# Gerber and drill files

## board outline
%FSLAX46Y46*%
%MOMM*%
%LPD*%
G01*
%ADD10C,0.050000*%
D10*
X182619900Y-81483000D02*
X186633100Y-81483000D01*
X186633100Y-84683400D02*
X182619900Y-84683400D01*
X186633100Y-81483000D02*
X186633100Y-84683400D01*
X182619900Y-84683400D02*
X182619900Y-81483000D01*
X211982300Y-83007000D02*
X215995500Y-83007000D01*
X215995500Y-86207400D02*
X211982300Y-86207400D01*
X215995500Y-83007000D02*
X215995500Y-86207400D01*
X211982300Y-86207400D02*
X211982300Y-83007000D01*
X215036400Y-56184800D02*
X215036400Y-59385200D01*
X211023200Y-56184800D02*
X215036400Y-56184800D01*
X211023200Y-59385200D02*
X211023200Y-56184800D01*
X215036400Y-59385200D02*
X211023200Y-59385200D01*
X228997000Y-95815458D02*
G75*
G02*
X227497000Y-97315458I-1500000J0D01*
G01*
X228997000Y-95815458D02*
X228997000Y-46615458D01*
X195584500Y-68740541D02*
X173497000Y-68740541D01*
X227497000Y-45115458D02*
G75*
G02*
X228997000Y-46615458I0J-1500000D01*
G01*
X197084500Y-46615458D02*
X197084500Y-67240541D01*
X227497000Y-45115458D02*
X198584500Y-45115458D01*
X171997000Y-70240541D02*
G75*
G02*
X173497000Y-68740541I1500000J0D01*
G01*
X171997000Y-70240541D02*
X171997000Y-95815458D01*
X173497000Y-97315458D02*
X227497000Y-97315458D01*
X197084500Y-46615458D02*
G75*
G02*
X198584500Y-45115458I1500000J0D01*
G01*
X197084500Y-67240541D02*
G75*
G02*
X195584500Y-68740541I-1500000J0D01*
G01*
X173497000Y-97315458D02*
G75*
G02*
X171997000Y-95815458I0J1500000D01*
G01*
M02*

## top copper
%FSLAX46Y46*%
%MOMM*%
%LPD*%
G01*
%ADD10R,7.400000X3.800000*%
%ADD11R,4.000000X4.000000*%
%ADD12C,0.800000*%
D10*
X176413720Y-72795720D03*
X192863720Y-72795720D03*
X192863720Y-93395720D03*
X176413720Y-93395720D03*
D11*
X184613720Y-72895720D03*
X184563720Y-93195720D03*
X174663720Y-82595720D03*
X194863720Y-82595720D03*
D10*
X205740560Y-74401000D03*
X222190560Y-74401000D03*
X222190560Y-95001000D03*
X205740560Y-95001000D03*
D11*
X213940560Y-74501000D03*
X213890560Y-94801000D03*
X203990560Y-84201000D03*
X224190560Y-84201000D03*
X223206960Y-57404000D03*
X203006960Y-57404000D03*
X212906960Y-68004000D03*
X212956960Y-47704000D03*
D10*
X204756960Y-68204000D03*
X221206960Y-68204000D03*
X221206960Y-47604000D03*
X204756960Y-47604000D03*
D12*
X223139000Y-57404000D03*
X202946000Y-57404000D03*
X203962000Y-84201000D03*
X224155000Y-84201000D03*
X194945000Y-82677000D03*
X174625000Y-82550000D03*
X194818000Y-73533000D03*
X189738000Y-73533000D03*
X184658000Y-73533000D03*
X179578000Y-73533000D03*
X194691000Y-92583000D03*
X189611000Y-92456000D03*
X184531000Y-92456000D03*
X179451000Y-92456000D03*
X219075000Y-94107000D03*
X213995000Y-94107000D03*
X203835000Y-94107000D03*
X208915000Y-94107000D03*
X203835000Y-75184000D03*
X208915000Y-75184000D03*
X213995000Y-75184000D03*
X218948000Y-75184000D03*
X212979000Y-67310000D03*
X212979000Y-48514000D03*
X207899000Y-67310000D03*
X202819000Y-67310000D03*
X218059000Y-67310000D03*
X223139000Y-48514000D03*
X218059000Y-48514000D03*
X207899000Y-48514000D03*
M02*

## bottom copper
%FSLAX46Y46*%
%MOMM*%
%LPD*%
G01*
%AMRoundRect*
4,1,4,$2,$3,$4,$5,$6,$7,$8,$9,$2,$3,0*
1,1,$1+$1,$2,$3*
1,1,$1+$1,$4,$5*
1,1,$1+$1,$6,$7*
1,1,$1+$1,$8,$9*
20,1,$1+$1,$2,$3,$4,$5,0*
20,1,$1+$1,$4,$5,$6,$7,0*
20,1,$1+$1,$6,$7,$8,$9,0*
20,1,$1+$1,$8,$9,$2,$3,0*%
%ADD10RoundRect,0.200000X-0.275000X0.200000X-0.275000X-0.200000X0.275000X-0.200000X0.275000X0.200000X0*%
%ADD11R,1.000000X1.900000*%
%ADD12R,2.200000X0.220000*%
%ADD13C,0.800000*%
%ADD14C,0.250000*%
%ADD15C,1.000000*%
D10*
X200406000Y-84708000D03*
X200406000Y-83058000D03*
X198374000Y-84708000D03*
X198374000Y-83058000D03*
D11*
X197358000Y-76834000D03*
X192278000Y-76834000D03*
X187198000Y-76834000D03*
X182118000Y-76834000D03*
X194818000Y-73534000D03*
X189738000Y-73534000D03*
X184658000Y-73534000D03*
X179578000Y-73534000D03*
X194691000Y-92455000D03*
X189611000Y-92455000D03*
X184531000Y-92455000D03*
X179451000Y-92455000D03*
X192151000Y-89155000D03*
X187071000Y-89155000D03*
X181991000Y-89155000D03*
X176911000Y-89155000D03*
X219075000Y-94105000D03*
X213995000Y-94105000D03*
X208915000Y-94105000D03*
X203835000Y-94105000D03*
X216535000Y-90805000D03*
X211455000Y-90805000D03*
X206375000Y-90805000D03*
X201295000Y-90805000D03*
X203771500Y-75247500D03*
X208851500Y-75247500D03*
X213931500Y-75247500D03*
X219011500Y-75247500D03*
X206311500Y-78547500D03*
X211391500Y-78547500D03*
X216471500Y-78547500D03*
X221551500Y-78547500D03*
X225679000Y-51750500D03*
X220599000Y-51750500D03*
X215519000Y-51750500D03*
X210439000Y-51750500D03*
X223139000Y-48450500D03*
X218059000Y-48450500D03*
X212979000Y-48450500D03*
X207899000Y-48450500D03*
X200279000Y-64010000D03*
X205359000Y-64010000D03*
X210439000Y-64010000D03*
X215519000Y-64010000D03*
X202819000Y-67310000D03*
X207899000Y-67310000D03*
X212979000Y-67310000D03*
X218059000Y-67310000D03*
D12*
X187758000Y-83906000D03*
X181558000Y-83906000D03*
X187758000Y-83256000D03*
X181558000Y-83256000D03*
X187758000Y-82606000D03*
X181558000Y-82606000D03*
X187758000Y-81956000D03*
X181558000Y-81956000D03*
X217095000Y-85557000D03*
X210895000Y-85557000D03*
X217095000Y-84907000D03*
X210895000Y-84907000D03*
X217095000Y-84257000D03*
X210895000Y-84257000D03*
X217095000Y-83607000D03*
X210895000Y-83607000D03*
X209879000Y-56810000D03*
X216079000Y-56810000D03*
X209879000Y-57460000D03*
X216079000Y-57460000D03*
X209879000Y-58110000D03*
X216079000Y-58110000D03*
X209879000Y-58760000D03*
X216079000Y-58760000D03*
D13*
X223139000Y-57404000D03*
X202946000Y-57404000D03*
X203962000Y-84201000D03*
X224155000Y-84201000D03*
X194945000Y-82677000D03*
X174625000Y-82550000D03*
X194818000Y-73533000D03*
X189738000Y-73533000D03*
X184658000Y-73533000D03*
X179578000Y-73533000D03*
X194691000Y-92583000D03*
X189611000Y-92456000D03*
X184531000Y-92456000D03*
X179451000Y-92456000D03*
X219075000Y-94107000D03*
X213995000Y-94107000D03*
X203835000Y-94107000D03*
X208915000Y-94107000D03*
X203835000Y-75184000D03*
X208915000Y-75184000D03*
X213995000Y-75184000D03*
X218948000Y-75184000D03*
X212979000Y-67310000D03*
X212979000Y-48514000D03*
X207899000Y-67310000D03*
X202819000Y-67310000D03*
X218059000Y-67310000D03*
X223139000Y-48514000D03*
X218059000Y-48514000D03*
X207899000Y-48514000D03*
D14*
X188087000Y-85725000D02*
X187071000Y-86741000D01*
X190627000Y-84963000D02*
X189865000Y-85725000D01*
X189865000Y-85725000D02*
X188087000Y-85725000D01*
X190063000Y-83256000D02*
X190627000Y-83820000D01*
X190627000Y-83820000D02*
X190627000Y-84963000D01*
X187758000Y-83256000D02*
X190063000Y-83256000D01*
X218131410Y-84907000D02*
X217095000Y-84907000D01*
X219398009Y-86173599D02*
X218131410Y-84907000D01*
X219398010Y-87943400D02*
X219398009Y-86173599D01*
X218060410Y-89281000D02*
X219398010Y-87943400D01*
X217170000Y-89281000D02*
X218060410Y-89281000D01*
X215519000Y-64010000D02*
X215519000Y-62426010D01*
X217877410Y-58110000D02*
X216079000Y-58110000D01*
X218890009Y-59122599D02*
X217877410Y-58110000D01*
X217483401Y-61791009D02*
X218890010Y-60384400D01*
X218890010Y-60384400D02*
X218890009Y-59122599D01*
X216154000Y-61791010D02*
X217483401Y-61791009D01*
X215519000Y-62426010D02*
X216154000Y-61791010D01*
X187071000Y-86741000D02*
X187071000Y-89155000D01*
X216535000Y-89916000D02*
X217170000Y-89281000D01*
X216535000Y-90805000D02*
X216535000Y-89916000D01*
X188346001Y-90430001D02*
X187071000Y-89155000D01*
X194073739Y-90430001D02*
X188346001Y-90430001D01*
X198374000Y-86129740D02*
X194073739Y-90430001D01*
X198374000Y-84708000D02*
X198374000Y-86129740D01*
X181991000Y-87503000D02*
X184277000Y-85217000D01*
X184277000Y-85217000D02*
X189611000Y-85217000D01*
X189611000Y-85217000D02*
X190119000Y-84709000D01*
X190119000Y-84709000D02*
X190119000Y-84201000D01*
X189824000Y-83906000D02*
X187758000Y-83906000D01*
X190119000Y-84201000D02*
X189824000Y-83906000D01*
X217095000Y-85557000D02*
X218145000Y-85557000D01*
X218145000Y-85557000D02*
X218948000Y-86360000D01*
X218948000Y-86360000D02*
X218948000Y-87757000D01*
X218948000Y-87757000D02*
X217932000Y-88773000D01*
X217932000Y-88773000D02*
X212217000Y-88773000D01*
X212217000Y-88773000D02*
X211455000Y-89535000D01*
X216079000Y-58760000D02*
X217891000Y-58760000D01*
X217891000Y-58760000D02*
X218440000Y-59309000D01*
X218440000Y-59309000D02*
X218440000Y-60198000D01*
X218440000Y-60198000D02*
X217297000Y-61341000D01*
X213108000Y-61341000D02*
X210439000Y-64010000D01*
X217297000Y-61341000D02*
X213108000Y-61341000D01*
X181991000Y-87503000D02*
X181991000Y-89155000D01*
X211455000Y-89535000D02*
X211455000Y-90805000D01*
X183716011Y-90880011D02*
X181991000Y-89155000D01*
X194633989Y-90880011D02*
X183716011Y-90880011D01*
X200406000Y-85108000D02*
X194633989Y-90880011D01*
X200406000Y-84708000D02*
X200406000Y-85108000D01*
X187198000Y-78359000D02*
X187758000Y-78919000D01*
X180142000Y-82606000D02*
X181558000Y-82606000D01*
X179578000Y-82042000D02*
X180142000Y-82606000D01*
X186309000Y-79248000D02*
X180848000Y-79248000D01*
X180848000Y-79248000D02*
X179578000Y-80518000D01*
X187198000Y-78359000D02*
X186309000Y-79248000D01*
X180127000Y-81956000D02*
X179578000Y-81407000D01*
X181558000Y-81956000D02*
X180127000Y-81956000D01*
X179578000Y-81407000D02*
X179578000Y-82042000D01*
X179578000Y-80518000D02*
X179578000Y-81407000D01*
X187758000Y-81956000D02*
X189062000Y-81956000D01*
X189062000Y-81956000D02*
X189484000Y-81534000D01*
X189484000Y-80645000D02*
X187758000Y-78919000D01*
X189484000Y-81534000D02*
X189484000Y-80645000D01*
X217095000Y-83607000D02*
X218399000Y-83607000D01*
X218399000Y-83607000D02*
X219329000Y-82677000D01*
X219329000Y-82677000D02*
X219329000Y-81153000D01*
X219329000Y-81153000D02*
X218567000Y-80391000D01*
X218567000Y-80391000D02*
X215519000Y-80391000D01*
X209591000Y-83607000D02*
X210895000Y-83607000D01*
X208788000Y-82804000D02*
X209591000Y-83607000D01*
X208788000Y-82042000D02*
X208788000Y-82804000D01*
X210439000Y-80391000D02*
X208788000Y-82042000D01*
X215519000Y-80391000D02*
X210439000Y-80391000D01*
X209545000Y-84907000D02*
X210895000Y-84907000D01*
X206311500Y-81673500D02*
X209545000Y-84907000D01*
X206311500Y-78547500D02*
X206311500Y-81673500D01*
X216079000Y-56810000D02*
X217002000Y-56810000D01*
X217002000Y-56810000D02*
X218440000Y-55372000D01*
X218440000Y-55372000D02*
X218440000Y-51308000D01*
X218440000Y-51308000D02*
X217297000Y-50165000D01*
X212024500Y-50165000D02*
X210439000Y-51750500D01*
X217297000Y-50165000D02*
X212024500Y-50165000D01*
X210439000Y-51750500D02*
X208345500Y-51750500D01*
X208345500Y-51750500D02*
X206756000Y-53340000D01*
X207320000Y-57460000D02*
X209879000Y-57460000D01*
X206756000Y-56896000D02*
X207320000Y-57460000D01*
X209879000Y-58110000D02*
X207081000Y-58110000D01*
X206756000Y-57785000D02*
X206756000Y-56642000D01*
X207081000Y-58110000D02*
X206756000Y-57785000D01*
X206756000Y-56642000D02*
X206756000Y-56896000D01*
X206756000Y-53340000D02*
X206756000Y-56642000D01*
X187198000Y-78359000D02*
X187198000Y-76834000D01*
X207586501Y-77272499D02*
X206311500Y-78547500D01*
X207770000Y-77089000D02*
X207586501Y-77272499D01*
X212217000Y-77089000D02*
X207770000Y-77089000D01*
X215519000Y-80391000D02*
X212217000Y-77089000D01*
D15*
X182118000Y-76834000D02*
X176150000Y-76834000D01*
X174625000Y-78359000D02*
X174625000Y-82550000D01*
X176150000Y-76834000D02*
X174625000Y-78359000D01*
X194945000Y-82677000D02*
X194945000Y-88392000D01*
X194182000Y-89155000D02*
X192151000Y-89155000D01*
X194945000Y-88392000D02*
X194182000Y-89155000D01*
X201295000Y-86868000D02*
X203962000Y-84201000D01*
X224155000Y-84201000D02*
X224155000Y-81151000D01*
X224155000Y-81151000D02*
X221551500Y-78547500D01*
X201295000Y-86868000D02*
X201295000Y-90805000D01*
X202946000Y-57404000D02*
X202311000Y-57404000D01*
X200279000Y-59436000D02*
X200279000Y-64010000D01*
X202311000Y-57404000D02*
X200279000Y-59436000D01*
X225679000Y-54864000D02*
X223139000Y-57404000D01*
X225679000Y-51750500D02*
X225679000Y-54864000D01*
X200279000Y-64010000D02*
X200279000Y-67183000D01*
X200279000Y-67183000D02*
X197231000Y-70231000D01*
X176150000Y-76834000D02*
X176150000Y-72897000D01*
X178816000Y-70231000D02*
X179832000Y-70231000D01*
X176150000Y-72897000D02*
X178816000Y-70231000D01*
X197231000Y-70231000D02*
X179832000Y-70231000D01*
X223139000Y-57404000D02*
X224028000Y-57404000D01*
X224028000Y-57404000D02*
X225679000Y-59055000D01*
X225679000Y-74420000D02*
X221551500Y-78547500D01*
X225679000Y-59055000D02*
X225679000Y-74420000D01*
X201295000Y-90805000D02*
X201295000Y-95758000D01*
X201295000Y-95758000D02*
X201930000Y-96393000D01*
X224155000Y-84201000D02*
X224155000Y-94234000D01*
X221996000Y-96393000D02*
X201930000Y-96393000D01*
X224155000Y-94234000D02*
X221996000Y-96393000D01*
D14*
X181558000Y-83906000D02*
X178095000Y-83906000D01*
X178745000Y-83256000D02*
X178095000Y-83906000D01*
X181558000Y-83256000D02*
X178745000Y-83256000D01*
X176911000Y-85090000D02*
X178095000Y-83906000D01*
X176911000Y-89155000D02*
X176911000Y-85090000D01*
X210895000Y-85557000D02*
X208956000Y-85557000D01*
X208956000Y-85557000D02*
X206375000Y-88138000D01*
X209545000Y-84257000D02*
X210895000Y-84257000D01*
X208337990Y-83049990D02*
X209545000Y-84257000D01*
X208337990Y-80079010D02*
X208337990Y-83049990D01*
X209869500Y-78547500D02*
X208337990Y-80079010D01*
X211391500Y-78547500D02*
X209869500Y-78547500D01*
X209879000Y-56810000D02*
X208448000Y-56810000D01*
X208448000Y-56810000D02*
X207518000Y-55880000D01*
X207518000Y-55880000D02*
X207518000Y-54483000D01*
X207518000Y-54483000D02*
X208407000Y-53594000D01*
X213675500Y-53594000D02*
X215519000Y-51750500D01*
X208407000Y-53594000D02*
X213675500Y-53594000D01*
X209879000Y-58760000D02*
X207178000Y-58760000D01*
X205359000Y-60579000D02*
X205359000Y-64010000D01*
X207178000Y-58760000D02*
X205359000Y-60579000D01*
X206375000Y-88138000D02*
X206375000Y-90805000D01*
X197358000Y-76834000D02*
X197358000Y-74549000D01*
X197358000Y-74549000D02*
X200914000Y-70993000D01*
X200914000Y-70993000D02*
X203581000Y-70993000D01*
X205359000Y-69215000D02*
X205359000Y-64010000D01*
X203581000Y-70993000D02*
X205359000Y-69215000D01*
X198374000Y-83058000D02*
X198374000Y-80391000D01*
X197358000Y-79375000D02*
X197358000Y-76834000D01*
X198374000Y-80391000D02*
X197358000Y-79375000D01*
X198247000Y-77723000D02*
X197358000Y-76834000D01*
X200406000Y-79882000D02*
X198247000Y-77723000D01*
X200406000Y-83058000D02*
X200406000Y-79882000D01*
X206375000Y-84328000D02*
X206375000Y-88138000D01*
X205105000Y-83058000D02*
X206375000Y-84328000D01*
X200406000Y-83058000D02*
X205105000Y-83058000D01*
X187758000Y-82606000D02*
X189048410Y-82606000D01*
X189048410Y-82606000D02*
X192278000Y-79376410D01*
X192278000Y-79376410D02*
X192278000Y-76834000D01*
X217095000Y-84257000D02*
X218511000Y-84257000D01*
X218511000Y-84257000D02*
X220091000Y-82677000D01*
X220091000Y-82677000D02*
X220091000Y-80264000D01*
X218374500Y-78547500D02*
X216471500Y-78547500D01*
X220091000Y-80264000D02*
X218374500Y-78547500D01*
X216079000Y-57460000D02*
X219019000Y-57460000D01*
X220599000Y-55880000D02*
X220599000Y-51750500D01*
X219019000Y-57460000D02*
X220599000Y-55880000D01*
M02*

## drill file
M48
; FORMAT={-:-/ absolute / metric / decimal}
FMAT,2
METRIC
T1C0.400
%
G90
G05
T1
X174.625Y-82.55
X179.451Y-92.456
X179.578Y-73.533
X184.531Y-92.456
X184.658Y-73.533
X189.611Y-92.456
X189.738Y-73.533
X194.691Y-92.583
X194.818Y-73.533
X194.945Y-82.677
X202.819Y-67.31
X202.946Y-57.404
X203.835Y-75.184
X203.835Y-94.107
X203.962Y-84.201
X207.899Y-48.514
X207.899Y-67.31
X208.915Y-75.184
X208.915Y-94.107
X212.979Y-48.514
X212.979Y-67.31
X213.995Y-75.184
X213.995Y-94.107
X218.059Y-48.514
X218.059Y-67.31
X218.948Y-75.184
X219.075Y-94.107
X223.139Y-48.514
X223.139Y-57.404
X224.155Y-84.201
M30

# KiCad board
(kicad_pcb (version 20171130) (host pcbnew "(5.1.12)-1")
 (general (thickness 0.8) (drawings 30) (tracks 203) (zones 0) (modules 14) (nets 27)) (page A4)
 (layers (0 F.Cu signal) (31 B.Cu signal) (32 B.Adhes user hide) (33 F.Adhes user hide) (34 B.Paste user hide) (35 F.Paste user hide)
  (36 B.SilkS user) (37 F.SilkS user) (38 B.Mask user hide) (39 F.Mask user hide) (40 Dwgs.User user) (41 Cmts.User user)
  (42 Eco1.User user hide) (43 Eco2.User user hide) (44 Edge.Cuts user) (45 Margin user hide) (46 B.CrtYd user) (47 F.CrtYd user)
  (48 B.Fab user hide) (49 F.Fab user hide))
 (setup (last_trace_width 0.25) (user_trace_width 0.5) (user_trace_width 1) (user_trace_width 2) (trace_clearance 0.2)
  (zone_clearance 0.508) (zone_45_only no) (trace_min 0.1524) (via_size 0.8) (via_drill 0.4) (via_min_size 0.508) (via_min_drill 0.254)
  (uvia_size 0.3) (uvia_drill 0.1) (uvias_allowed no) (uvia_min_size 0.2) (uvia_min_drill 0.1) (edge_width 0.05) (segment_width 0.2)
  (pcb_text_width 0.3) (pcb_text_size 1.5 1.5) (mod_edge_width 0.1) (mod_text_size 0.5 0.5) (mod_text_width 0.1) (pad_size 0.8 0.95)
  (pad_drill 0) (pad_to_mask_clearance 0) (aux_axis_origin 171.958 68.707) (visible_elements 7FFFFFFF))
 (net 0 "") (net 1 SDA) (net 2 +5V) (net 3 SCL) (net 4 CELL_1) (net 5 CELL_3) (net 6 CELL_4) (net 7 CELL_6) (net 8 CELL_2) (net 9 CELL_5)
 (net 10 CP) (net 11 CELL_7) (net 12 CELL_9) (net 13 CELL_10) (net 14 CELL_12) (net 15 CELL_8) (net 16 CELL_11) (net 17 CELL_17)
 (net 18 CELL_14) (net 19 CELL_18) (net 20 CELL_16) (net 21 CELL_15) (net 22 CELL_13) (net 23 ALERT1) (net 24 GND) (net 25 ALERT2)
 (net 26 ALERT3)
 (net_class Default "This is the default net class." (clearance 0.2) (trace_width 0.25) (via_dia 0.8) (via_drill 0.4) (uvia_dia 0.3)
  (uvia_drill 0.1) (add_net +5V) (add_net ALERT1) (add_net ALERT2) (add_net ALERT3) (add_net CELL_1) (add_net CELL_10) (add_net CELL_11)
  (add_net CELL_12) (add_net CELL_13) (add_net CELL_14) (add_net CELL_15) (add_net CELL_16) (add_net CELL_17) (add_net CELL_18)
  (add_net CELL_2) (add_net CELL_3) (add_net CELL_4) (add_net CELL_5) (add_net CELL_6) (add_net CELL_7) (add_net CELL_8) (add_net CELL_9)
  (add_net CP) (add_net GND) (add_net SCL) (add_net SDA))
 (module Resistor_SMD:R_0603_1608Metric (layer B.Cu) (at 200.406 83.883 270)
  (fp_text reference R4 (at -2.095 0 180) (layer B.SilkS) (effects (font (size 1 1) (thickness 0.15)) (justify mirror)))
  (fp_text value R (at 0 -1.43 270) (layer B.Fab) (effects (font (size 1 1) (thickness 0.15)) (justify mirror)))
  (pad 2 smd roundrect (at 0.825 0 270) (size 0.8 0.95) (layers B.Cu B.Paste B.Mask) (roundrect_rratio 0.25) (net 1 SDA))
  (pad 1 smd roundrect (at -0.825 0 270) (size 0.8 0.95) (layers B.Cu B.Paste B.Mask) (roundrect_rratio 0.25) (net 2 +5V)))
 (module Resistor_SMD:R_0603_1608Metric (layer B.Cu) (at 198.374 83.883 270)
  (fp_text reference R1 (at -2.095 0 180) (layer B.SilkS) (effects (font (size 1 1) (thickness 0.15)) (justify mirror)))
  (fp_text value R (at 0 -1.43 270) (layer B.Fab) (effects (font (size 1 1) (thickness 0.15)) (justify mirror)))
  (pad 2 smd roundrect (at 0.825 0 270) (size 0.8 0.95) (layers B.Cu B.Paste B.Mask) (roundrect_rratio 0.25) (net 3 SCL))
  (pad 1 smd roundrect (at -0.825 0 270) (size 0.8 0.95) (layers B.Cu B.Paste B.Mask) (roundrect_rratio 0.25) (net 2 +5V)))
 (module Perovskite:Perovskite (layer F.Cu) (at 171.86372 70.19572)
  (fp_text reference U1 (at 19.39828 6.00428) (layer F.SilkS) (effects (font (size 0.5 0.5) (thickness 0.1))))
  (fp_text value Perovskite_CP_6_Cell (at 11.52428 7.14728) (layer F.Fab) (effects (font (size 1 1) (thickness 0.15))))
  (pad 1 smd rect (at 4.55 2.6) (size 7.4 3.8) (layers F.Cu F.Paste F.Mask) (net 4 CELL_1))
  (pad 3 smd rect (at 21 2.6) (size 7.4 3.8) (layers F.Cu F.Paste F.Mask) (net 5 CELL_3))
  (pad 4 smd rect (at 21 23.2) (size 7.4 3.8) (layers F.Cu F.Paste F.Mask) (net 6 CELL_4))
  (pad 6 smd rect (at 4.55 23.2) (size 7.4 3.8) (layers F.Cu F.Paste F.Mask) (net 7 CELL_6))
  (pad 2 smd rect (at 12.75 2.7) (size 4 4) (layers F.Cu F.Paste F.Mask) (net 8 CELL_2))
  (pad 5 smd rect (at 12.7 23) (size 4 4) (layers F.Cu F.Paste F.Mask) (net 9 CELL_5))
  (pad 7 smd rect (at 2.8 12.4) (size 4 4) (layers F.Cu F.Paste F.Mask) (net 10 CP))
  (pad 7 smd rect (at 23 12.4) (size 4 4) (layers F.Cu F.Paste F.Mask) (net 10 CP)))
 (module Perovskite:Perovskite (layer F.Cu) (at 201.19056 71.801)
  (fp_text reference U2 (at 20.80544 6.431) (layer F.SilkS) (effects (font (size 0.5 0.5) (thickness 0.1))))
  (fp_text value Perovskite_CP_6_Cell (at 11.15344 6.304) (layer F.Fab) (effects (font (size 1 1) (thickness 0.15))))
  (pad 1 smd rect (at 4.55 2.6) (size 7.4 3.8) (layers F.Cu F.Paste F.Mask) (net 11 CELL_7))
  (pad 3 smd rect (at 21 2.6) (size 7.4 3.8) (layers F.Cu F.Paste F.Mask) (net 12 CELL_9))
  (pad 4 smd rect (at 21 23.2) (size 7.4 3.8) (layers F.Cu F.Paste F.Mask) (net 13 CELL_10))
  (pad 6 smd rect (at 4.55 23.2) (size 7.4 3.8) (layers F.Cu F.Paste F.Mask) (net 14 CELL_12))
  (pad 2 smd rect (at 12.75 2.7) (size 4 4) (layers F.Cu F.Paste F.Mask) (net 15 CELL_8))
  (pad 5 smd rect (at 12.7 23) (size 4 4) (layers F.Cu F.Paste F.Mask) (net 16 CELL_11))
  (pad 7 smd rect (at 2.8 12.4) (size 4 4) (layers F.Cu F.Paste F.Mask) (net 10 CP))
  (pad 7 smd rect (at 23 12.4) (size 4 4) (layers F.Cu F.Paste F.Mask) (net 10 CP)))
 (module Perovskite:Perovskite (layer F.Cu) (at 200.20696 45.004)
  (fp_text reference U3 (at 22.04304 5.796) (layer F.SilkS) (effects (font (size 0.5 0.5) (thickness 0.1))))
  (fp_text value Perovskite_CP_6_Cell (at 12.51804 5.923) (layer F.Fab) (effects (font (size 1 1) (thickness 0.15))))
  (pad 7 smd rect (at 23 12.4) (size 4 4) (layers F.Cu F.Paste F.Mask) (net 10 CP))
  (pad 7 smd rect (at 2.8 12.4) (size 4 4) (layers F.Cu F.Paste F.Mask) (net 10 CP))
  (pad 5 smd rect (at 12.7 23) (size 4 4) (layers F.Cu F.Paste F.Mask) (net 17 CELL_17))
  (pad 2 smd rect (at 12.75 2.7) (size 4 4) (layers F.Cu F.Paste F.Mask) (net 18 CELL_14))
  (pad 6 smd rect (at 4.55 23.2) (size 7.4 3.8) (layers F.Cu F.Paste F.Mask) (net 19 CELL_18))
  (pad 4 smd rect (at 21 23.2) (size 7.4 3.8) (layers F.Cu F.Paste F.Mask) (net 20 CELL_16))
  (pad 3 smd rect (at 21 2.6) (size 7.4 3.8) (layers F.Cu F.Paste F.Mask) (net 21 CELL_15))
  (pad 1 smd rect (at 4.55 2.6) (size 7.4 3.8) (layers F.Cu F.Paste F.Mask) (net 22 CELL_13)))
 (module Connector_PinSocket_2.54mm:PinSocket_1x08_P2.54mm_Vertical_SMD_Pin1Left (layer B.Cu) (at 188.468 75.184 90)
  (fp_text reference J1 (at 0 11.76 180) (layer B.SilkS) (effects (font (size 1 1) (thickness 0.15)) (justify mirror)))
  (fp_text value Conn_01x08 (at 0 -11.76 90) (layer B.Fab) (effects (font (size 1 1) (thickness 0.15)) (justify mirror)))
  (pad 1 smd rect (at -1.65 8.89 90) (size 1.9 1) (layers B.Cu B.Paste B.Mask) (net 2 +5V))
  (pad 3 smd rect (at -1.65 3.81 90) (size 1.9 1) (layers B.Cu B.Paste B.Mask) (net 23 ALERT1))
  (pad 5 smd rect (at -1.65 -1.27 90) (size 1.9 1) (layers B.Cu B.Paste B.Mask) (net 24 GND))
  (pad 7 smd rect (at -1.65 -6.35 90) (size 1.9 1) (layers B.Cu B.Paste B.Mask) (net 10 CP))
  (pad 2 smd rect (at 1.65 6.35 90) (size 1.9 1) (layers B.Cu B.Paste B.Mask) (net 5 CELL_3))
  (pad 4 smd rect (at 1.65 1.27 90) (size 1.9 1) (layers B.Cu B.Paste B.Mask) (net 5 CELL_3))
  (pad 6 smd rect (at 1.65 -3.81 90) (size 1.9 1) (layers B.Cu B.Paste B.Mask) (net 8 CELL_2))
  (pad 8 smd rect (at 1.65 -8.89 90) (size 1.9 1) (layers B.Cu B.Paste B.Mask) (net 4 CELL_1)))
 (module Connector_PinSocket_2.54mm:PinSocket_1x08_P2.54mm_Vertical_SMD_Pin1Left (layer B.Cu) (at 185.801 90.805 270)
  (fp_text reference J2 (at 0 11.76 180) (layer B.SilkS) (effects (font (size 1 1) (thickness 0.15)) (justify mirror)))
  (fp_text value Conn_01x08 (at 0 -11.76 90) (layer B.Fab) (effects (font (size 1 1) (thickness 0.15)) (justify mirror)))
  (pad 8 smd rect (at 1.65 -8.89 270) (size 1.9 1) (layers B.Cu B.Paste B.Mask) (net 6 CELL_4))
  (pad 6 smd rect (at 1.65 -3.81 270) (size 1.9 1) (layers B.Cu B.Paste B.Mask) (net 6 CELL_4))
  (pad 4 smd rect (at 1.65 1.27 270) (size 1.9 1) (layers B.Cu B.Paste B.Mask) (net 9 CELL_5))
  (pad 2 smd rect (at 1.65 6.35 270) (size 1.9 1) (layers B.Cu B.Paste B.Mask) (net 7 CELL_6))
  (pad 7 smd rect (at -1.65 -6.35 270) (size 1.9 1) (layers B.Cu B.Paste B.Mask) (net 10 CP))
  (pad 5 smd rect (at -1.65 -1.27 270) (size 1.9 1) (layers B.Cu B.Paste B.Mask) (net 3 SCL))
  (pad 3 smd rect (at -1.65 3.81 270) (size 1.9 1) (layers B.Cu B.Paste B.Mask) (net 1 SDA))
  (pad 1 smd rect (at -1.65 8.89 270) (size 1.9 1) (layers B.Cu B.Paste B.Mask) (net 2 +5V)))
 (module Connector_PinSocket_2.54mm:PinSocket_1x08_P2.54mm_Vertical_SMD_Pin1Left (layer B.Cu) (at 210.185 92.455 90)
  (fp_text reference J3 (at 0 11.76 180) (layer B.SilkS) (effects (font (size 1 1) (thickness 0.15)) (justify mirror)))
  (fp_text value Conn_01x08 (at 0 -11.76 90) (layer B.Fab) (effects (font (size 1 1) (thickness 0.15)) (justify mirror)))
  (pad 1 smd rect (at -1.65 8.89 90) (size 1.9 1) (layers B.Cu B.Paste B.Mask) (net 13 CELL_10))
  (pad 3 smd rect (at -1.65 3.81 90) (size 1.9 1) (layers B.Cu B.Paste B.Mask) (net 16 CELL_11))
  (pad 5 smd rect (at -1.65 -1.27 90) (size 1.9 1) (layers B.Cu B.Paste B.Mask) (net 14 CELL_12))
  (pad 7 smd rect (at -1.65 -6.35 90) (size 1.9 1) (layers B.Cu B.Paste B.Mask) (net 14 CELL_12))
  (pad 2 smd rect (at 1.65 6.35 90) (size 1.9 1) (layers B.Cu B.Paste B.Mask) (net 3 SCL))
  (pad 4 smd rect (at 1.65 1.27 90) (size 1.9 1) (layers B.Cu B.Paste B.Mask) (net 1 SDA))
  (pad 6 smd rect (at 1.65 -3.81 90) (size 1.9 1) (layers B.Cu B.Paste B.Mask) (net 2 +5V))
  (pad 8 smd rect (at 1.65 -8.89 90) (size 1.9 1) (layers B.Cu B.Paste B.Mask) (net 10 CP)))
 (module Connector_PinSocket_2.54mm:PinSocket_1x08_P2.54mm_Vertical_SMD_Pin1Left (layer B.Cu) (at 212.6615 76.8975 90)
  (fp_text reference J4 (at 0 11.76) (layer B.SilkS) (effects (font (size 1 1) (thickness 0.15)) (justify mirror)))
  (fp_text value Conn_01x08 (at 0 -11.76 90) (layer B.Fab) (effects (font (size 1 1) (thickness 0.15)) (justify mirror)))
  (pad 8 smd rect (at 1.65 -8.89 90) (size 1.9 1) (layers B.Cu B.Paste B.Mask) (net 11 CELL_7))
  (pad 6 smd rect (at 1.65 -3.81 90) (size 1.9 1) (layers B.Cu B.Paste B.Mask) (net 11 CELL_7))
  (pad 4 smd rect (at 1.65 1.27 90) (size 1.9 1) (layers B.Cu B.Paste B.Mask) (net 15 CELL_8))
  (pad 2 smd rect (at 1.65 6.35 90) (size 1.9 1) (layers B.Cu B.Paste B.Mask) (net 12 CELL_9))
  (pad 7 smd rect (at -1.65 -6.35 90) (size 1.9 1) (layers B.Cu B.Paste B.Mask) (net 24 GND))
  (pad 5 smd rect (at -1.65 -1.27 90) (size 1.9 1) (layers B.Cu B.Paste B.Mask) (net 2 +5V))
  (pad 3 smd rect (at -1.65 3.81 90) (size 1.9 1) (layers B.Cu B.Paste B.Mask) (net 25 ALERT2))
  (pad 1 smd rect (at -1.65 8.89 90) (size 1.9 1) (layers B.Cu B.Paste B.Mask) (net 10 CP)))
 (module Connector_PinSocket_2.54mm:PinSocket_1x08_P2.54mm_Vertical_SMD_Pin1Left (layer B.Cu) (at 216.789 50.1005 90)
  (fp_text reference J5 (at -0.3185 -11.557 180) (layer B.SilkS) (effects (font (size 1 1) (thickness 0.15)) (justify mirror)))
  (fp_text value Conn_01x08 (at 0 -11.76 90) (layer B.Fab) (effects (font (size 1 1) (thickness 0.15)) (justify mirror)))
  (pad 1 smd rect (at -1.65 8.89 90) (size 1.9 1) (layers B.Cu B.Paste B.Mask) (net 10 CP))
  (pad 3 smd rect (at -1.65 3.81 90) (size 1.9 1) (layers B.Cu B.Paste B.Mask) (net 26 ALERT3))
  (pad 5 smd rect (at -1.65 -1.27 90) (size 1.9 1) (layers B.Cu B.Paste B.Mask) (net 2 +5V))
  (pad 7 smd rect (at -1.65 -6.35 90) (size 1.9 1) (layers B.Cu B.Paste B.Mask) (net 24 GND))
  (pad 2 smd rect (at 1.65 6.35 90) (size 1.9 1) (layers B.Cu B.Paste B.Mask) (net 21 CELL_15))
  (pad 4 smd rect (at 1.65 1.27 90) (size 1.9 1) (layers B.Cu B.Paste B.Mask) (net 21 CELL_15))
  (pad 6 smd rect (at 1.65 -3.81 90) (size 1.9 1) (layers B.Cu B.Paste B.Mask) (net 18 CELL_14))
  (pad 8 smd rect (at 1.65 -8.89 90) (size 1.9 1) (layers B.Cu B.Paste B.Mask) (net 22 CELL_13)))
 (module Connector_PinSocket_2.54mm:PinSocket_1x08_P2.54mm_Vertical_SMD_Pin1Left (layer B.Cu) (at 209.169 65.66 90)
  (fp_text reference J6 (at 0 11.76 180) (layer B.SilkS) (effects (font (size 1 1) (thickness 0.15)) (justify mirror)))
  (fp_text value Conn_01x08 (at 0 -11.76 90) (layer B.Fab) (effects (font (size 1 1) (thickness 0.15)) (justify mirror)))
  (pad 8 smd rect (at 1.65 -8.89 90) (size 1.9 1) (layers B.Cu B.Paste B.Mask) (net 10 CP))
  (pad 6 smd rect (at 1.65 -3.81 90) (size 1.9 1) (layers B.Cu B.Paste B.Mask) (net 2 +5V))
  (pad 4 smd rect (at 1.65 1.27 90) (size 1.9 1) (layers B.Cu B.Paste B.Mask) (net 1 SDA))
  (pad 2 smd rect (at 1.65 6.35 90) (size 1.9 1) (layers B.Cu B.Paste B.Mask) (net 3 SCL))
  (pad 7 smd rect (at -1.65 -6.35 90) (size 1.9 1) (layers B.Cu B.Paste B.Mask) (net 19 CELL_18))
  (pad 5 smd rect (at -1.65 -1.27 90) (size 1.9 1) (layers B.Cu B.Paste B.Mask) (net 19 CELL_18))
  (pad 3 smd rect (at -1.65 3.81 90) (size 1.9 1) (layers B.Cu B.Paste B.Mask) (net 17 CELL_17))
  (pad 1 smd rect (at -1.65 8.89 90) (size 1.9 1) (layers B.Cu B.Paste B.Mask) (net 20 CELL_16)))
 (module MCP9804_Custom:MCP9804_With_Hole (layer B.Cu) (at 184.658 82.931)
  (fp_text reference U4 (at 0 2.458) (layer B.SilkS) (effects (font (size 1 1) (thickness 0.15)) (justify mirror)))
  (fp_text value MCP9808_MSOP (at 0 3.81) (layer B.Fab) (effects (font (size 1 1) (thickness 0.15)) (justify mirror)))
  (pad 1 smd rect (at 3.1 0.975 90) (size 0.22 2.2) (layers B.Cu B.Paste B.Mask) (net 1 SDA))
  (pad 8 smd rect (at -3.1 0.975 90) (size 0.22 2.2) (layers B.Cu B.Paste B.Mask) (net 2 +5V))
  (pad 2 smd rect (at 3.1 0.325 90) (size 0.22 2.2) (layers B.Cu B.Paste B.Mask) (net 3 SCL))
  (pad 7 smd rect (at -3.1 0.325 90) (size 0.22 2.2) (layers B.Cu B.Paste B.Mask) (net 2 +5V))
  (pad 3 smd rect (at 3.1 -0.325 90) (size 0.22 2.2) (layers B.Cu B.Paste B.Mask) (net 23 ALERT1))
  (pad 6 smd rect (at -3.1 -0.325 90) (size 0.22 2.2) (layers B.Cu B.Paste B.Mask) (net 24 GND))
  (pad 4 smd rect (at 3.1 -0.975 90) (size 0.22 2.2) (layers B.Cu B.Paste B.Mask) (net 24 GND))
  (pad 5 smd rect (at -3.1 -0.975 90) (size 0.22 2.2) (layers B.Cu B.Paste B.Mask) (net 24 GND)))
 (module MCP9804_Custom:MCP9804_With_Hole (layer B.Cu) (at 213.995 84.582)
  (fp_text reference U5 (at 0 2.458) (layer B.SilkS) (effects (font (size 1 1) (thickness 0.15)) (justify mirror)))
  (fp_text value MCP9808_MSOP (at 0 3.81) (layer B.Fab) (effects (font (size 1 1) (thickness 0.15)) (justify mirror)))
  (pad 1 smd rect (at 3.1 0.975 90) (size 0.22 2.2) (layers B.Cu B.Paste B.Mask) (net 1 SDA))
  (pad 8 smd rect (at -3.1 0.975 90) (size 0.22 2.2) (layers B.Cu B.Paste B.Mask) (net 2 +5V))
  (pad 2 smd rect (at 3.1 0.325 90) (size 0.22 2.2) (layers B.Cu B.Paste B.Mask) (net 3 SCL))
  (pad 7 smd rect (at -3.1 0.325 90) (size 0.22 2.2) (layers B.Cu B.Paste B.Mask) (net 24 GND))
  (pad 3 smd rect (at 3.1 -0.325 90) (size 0.22 2.2) (layers B.Cu B.Paste B.Mask) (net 25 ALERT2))
  (pad 6 smd rect (at -3.1 -0.325 90) (size 0.22 2.2) (layers B.Cu B.Paste B.Mask) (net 2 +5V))
  (pad 4 smd rect (at 3.1 -0.975 90) (size 0.22 2.2) (layers B.Cu B.Paste B.Mask) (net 24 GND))
  (pad 5 smd rect (at -3.1 -0.975 90) (size 0.22 2.2) (layers B.Cu B.Paste B.Mask) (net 24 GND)))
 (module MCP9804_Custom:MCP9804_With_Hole (layer B.Cu) (at 212.979 57.785)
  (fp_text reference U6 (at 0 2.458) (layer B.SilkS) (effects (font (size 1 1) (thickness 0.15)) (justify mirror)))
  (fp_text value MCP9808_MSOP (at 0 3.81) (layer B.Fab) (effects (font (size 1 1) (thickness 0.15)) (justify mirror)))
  (pad 5 smd rect (at -3.1 -0.975 90) (size 0.22 2.2) (layers B.Cu B.Paste B.Mask) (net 2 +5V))
  (pad 4 smd rect (at 3.1 -0.975 90) (size 0.22 2.2) (layers B.Cu B.Paste B.Mask) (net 24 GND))
  (pad 6 smd rect (at -3.1 -0.325 90) (size 0.22 2.2) (layers B.Cu B.Paste B.Mask) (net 24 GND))
  (pad 3 smd rect (at 3.1 -0.325 90) (size 0.22 2.2) (layers B.Cu B.Paste B.Mask) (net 26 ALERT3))
  (pad 7 smd rect (at -3.1 0.325 90) (size 0.22 2.2) (layers B.Cu B.Paste B.Mask) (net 24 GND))
  (pad 2 smd rect (at 3.1 0.325 90) (size 0.22 2.2) (layers B.Cu B.Paste B.Mask) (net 3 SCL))
  (pad 8 smd rect (at -3.1 0.975 90) (size 0.22 2.2) (layers B.Cu B.Paste B.Mask) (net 2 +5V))
  (pad 1 smd rect (at 3.1 0.975 90) (size 0.22 2.2) (layers B.Cu B.Paste B.Mask) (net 1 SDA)))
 (gr_line (start 182.6199 81.483) (end 186.6331 81.483) (layer Edge.Cuts) (width 0.05))
 (gr_line (start 186.6331 84.6834) (end 182.6199 84.6834) (layer Edge.Cuts) (width 0.05))
 (gr_line (start 186.6331 81.483) (end 186.6331 84.6834) (layer Edge.Cuts) (width 0.05))
 (gr_line (start 182.6199 84.6834) (end 182.6199 81.483) (layer Edge.Cuts) (width 0.05))
 (gr_line (start 211.9823 83.007) (end 215.9955 83.007) (layer Edge.Cuts) (width 0.05))
 (gr_line (start 215.9955 86.2074) (end 211.9823 86.2074) (layer Edge.Cuts) (width 0.05))
 (gr_line (start 215.9955 83.007) (end 215.9955 86.2074) (layer Edge.Cuts) (width 0.05))
 (gr_line (start 211.9823 86.2074) (end 211.9823 83.007) (layer Edge.Cuts) (width 0.05))
 (gr_line (start 215.0364 56.1848) (end 215.0364 59.3852) (layer Edge.Cuts) (width 0.05))
 (gr_line (start 211.0232 56.1848) (end 215.0364 56.1848) (layer Edge.Cuts) (width 0.05))
 (gr_line (start 211.0232 59.3852) (end 211.0232 56.1848) (layer Edge.Cuts) (width 0.05))
 (gr_line (start 215.0364 59.3852) (end 211.0232 59.3852) (layer Edge.Cuts) (width 0.05))
 (gr_arc (start 227.497 95.815458) (end 227.497 97.315458) (angle -90) (layer Edge.Cuts) (width 0.05))
 (gr_line (start 228.997 95.815458) (end 228.997 46.615458) (layer Edge.Cuts) (width 0.05))
 (gr_line (start 195.5845 68.740541) (end 173.497 68.740541) (layer Edge.Cuts) (width 0.05))
 (gr_arc (start 227.497 46.615458) (end 228.997 46.615458) (angle -90) (layer Edge.Cuts) (width 0.05))
 (gr_line (start 197.0845 46.615458) (end 197.0845 67.240541) (layer Edge.Cuts) (width 0.05))
 (gr_line (start 227.497 45.115458) (end 198.5845 45.115458) (layer Edge.Cuts) (width 0.05))
 (gr_arc (start 173.497 70.240541) (end 173.497 68.740541) (angle -90) (layer Edge.Cuts) (width 0.05))
 (gr_line (start 171.997 70.240541) (end 171.997 95.815458) (layer Edge.Cuts) (width 0.05))
 (gr_line (start 173.497 97.315458) (end 227.497 97.315458) (layer Edge.Cuts) (width 0.05))
 (gr_arc (start 198.5845 46.615458) (end 198.5845 45.115458) (angle -90) (layer Edge.Cuts) (width 0.05))
 (gr_arc (start 195.5845 67.240541) (end 195.5845 68.740541) (angle -90) (layer Edge.Cuts) (width 0.05))
 (gr_arc (start 173.497 95.815458) (end 171.997 95.815458) (angle -90) (layer Edge.Cuts) (width 0.05))
 (segment (start 188.087 85.725) (end 187.071 86.741) (width 0.25) (layer B.Cu) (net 3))
 (segment (start 190.627 84.963) (end 189.865 85.725) (width 0.25) (layer B.Cu) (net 3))
 (segment (start 189.865 85.725) (end 188.087 85.725) (width 0.25) (layer B.Cu) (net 3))
 (segment (start 190.063 83.256) (end 190.627 83.82) (width 0.25) (layer B.Cu) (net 3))
 (segment (start 190.627 83.82) (end 190.627 84.963) (width 0.25) (layer B.Cu) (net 3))
 (segment (start 187.758 83.256) (end 190.063 83.256) (width 0.25) (layer B.Cu) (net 3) (status 10))
 (segment (start 218.13141 84.907) (end 217.095 84.907) (width 0.25) (layer B.Cu) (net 3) (status 30))
 (segment (start 219.398009 86.173599) (end 218.13141 84.907) (width 0.25) (layer B.Cu) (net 3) (status 20))
 (segment (start 219.39801 87.9434) (end 219.398009 86.173599) (width 0.25) (layer B.Cu) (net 3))
 (segment (start 218.06041 89.281) (end 219.39801 87.9434) (width 0.25) (layer B.Cu) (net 3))
 (segment (start 217.17 89.281) (end 218.06041 89.281) (width 0.25) (layer B.Cu) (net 3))
 (segment (start 215.519 64.01) (end 215.519 62.42601) (width 0.25) (layer B.Cu) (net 3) (status 10))
 (segment (start 217.87741 58.11) (end 216.079 58.11) (width 0.25) (layer B.Cu) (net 3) (status 20))
 (segment (start 218.890009 59.122599) (end 217.87741 58.11) (width 0.25) (layer B.Cu) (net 3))
 (segment (start 217.483401 61.791009) (end 218.89001 60.3844) (width 0.25) (layer B.Cu) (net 3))
 (segment (start 218.89001 60.3844) (end 218.890009 59.122599) (width 0.25) (layer B.Cu) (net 3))
 (segment (start 216.154 61.79101) (end 217.483401 61.791009) (width 0.25) (layer B.Cu) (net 3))
 (segment (start 215.519 62.42601) (end 216.154 61.79101) (width 0.25) (layer B.Cu) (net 3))
 (segment (start 187.071 86.741) (end 187.071 89.155) (width 0.25) (layer B.Cu) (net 3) (status 20))
 (segment (start 216.535 89.916) (end 217.17 89.281) (width 0.25) (layer B.Cu) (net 3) (status 10))
 (segment (start 216.535 90.805) (end 216.535 89.916) (width 0.25) (layer B.Cu) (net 3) (status 30))
 (segment (start 188.346001 90.430001) (end 187.071 89.155) (width 0.25) (layer B.Cu) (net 3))
 (segment (start 194.073739 90.430001) (end 188.346001 90.430001) (width 0.25) (layer B.Cu) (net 3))
 (segment (start 198.374 86.12974) (end 194.073739 90.430001) (width 0.25) (layer B.Cu) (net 3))
 (segment (start 198.374 84.708) (end 198.374 86.12974) (width 0.25) (layer B.Cu) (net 3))
 (segment (start 181.991 87.503) (end 184.277 85.217) (width 0.25) (layer B.Cu) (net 1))
 (segment (start 184.277 85.217) (end 189.611 85.217) (width 0.25) (layer B.Cu) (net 1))
 (segment (start 189.611 85.217) (end 190.119 84.709) (width 0.25) (layer B.Cu) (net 1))
 (segment (start 190.119 84.709) (end 190.119 84.201) (width 0.25) (layer B.Cu) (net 1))
 (segment (start 189.824 83.906) (end 187.758 83.906) (width 0.25) (layer B.Cu) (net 1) (status 20))
 (segment (start 190.119 84.201) (end 189.824 83.906) (width 0.25) (layer B.Cu) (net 1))
 (segment (start 217.095 85.557) (end 218.145 85.557) (width 0.25) (layer B.Cu) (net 1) (status 30))
 (segment (start 218.145 85.557) (end 218.948 86.36) (width 0.25) (layer B.Cu) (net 1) (status 10))
 (segment (start 218.948 86.36) (end 218.948 87.757) (width 0.25) (layer B.Cu) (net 1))
 (segment (start 218.948 87.757) (end 217.932 88.773) (width 0.25) (layer B.Cu) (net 1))
 (segment (start 217.932 88.773) (end 212.217 88.773) (width 0.25) (layer B.Cu) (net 1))
 (segment (start 212.217 88.773) (end 211.455 89.535) (width 0.25) (layer B.Cu) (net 1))
 (segment (start 216.079 58.76) (end 217.891 58.76) (width 0.25) (layer B.Cu) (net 1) (status 10))
 (segment (start 217.891 58.76) (end 218.44 59.309) (width 0.25) (layer B.Cu) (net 1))
 (segment (start 218.44 59.309) (end 218.44 60.198) (width 0.25) (layer B.Cu) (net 1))
 (segment (start 218.44 60.198) (end 217.297 61.341) (width 0.25) (layer B.Cu) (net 1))
 (segment (start 213.108 61.341) (end 210.439 64.01) (width 0.25) (layer B.Cu) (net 1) (status 20))
 (segment (start 217.297 61.341) (end 213.108 61.341) (width 0.25) (layer B.Cu) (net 1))
 (segment (start 181.991 87.503) (end 181.991 89.155) (width 0.25) (layer B.Cu) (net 1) (status 20))
 (segment (start 211.455 89.535) (end 211.455 90.805) (width 0.25) (layer B.Cu) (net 1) (status 20))
 (segment (start 183.716011 90.880011) (end 181.991 89.155) (width 0.25) (layer B.Cu) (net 1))
 (segment (start 194.633989 90.880011) (end 183.716011 90.880011) (width 0.25) (layer B.Cu) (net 1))
 (segment (start 200.406 85.108) (end 194.633989 90.880011) (width 0.25) (layer B.Cu) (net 1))
 (segment (start 200.406 84.708) (end 200.406 85.108) (width 0.25) (layer B.Cu) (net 1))
 (segment (start 187.198 78.359) (end 187.758 78.919) (width 0.25) (layer B.Cu) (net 24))
 (segment (start 180.142 82.606) (end 181.558 82.606) (width 0.25) (layer B.Cu) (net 24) (status 20))
 (segment (start 179.578 82.042) (end 180.142 82.606) (width 0.25) (layer B.Cu) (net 24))
 (segment (start 186.309 79.248) (end 180.848 79.248) (width 0.25) (layer B.Cu) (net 24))
 (segment (start 180.848 79.248) (end 179.578 80.518) (width 0.25) (layer B.Cu) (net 24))
 (segment (start 187.198 78.359) (end 186.309 79.248) (width 0.25) (layer B.Cu) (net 24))
 (segment (start 180.127 81.956) (end 179.578 81.407) (width 0.25) (layer B.Cu) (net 24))
 (segment (start 181.558 81.956) (end 180.127 81.956) (width 0.25) (layer B.Cu) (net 24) (status 10))
 (segment (start 179.578 81.407) (end 179.578 82.042) (width 0.25) (layer B.Cu) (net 24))
 (segment (start 179.578 80.518) (end 179.578 81.407) (width 0.25) (layer B.Cu) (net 24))
 (segment (start 187.758 81.956) (end 189.062 81.956) (width 0.25) (layer B.Cu) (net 24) (status 10))
 (segment (start 189.062 81.956) (end 189.484 81.534) (width 0.25) (layer B.Cu) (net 24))
 (segment (start 189.484 80.645) (end 187.758 78.919) (width 0.25) (layer B.Cu) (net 24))
 (segment (start 189.484 81.534) (end 189.484 80.645) (width 0.25) (layer B.Cu) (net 24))
 (segment (start 217.095 83.607) (end 218.399 83.607) (width 0.25) (layer B.Cu) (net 24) (status 10))
 (segment (start 218.399 83.607) (end 219.329 82.677) (width 0.25) (layer B.Cu) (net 24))
 (segment (start 219.329 82.677) (end 219.329 81.153) (width 0.25) (layer B.Cu) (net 24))
 (segment (start 219.329 81.153) (end 218.567 80.391) (width 0.25) (layer B.Cu) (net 24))
 (segment (start 218.567 80.391) (end 215.519 80.391) (width 0.25) (layer B.Cu) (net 24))
 (segment (start 209.591 83.607) (end 210.895 83.607) (width 0.25) (layer B.Cu) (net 24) (status 20))
 (segment (start 208.788 82.804) (end 209.591 83.607) (width 0.25) (layer B.Cu) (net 24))
 (segment (start 208.788 82.042) (end 208.788 82.804) (width 0.25) (layer B.Cu) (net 24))
 (segment (start 210.439 80.391) (end 208.788 82.042) (width 0.25) (layer B.Cu) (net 24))
 (segment (start 215.519 80.391) (end 210.439 80.391) (width 0.25) (layer B.Cu) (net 24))
 (segment (start 209.545 84.907) (end 210.895 84.907) (width 0.25) (layer B.Cu) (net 24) (status 20))
 (segment (start 206.3115 81.6735) (end 209.545 84.907) (width 0.25) (layer B.Cu) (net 24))
 (segment (start 206.3115 78.5475) (end 206.3115 81.6735) (width 0.25) (layer B.Cu) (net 24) (status 10))
 (segment (start 216.079 56.81) (end 217.002 56.81) (width 0.25) (layer B.Cu) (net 24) (status 30))
 (segment (start 217.002 56.81) (end 218.44 55.372) (width 0.25) (layer B.Cu) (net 24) (status 10))
 (segment (start 218.44 55.372) (end 218.44 51.308) (width 0.25) (layer B.Cu) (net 24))
 (segment (start 218.44 51.308) (end 217.297 50.165) (width 0.25) (layer B.Cu) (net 24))
 (segment (start 212.0245 50.165) (end 210.439 51.7505) (width 0.25) (layer B.Cu) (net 24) (status 20))
 (segment (start 217.297 50.165) (end 212.0245 50.165) (width 0.25) (layer B.Cu) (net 24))
 (segment (start 210.439 51.7505) (end 208.3455 51.7505) (width 0.25) (layer B.Cu) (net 24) (status 10))
 (segment (start 208.3455 51.7505) (end 206.756 53.34) (width 0.25) (layer B.Cu) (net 24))
 (segment (start 207.32 57.46) (end 209.879 57.46) (width 0.25) (layer B.Cu) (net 24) (status 20))
 (segment (start 206.756 56.896) (end 207.32 57.46) (width 0.25) (layer B.Cu) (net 24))
 (segment (start 209.879 58.11) (end 207.081 58.11) (width 0.25) (layer B.Cu) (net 24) (status 10))
 (segment (start 206.756 57.785) (end 206.756 56.642) (width 0.25) (layer B.Cu) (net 24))
 (segment (start 207.081 58.11) (end 206.756 57.785) (width 0.25) (layer B.Cu) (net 24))
 (segment (start 206.756 56.642) (end 206.756 56.896) (width 0.25) (layer B.Cu) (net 24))
 (segment (start 206.756 53.34) (end 206.756 56.642) (width 0.25) (layer B.Cu) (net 24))
 (segment (start 187.198 78.359) (end 187.198 76.834) (width 0.25) (layer B.Cu) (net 24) (status 20))
 (segment (start 207.586501 77.272499) (end 206.3115 78.5475) (width 0.25) (layer B.Cu) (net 24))
 (segment (start 207.77 77.089) (end 207.586501 77.272499) (width 0.25) (layer B.Cu) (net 24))
 (segment (start 212.217 77.089) (end 207.77 77.089) (width 0.25) (layer B.Cu) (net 24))
 (segment (start 215.519 80.391) (end 212.217 77.089) (width 0.25) (layer B.Cu) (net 24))
 (via (at 223.139 57.404) (size 0.8) (drill 0.4) (layers F.Cu B.Cu) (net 10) (status 30))
 (via (at 202.946 57.404) (size 0.8) (drill 0.4) (layers F.Cu B.Cu) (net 10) (status 30))
 (via (at 203.962 84.201) (size 0.8) (drill 0.4) (layers F.Cu B.Cu) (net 10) (status 30))
 (via (at 224.155 84.201) (size 0.8) (drill 0.4) (layers F.Cu B.Cu) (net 10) (status 30))
 (via (at 194.945 82.677) (size 0.8) (drill 0.4) (layers F.Cu B.Cu) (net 10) (status 30))
 (via (at 174.625 82.55) (size 0.8) (drill 0.4) (layers F.Cu B.Cu) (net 10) (status 30))
 (segment (start 182.118 76.834) (end 176.15 76.834) (width 1) (layer B.Cu) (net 10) (status 10))
 (segment (start 174.625 78.359) (end 174.625 82.55) (width 1) (layer B.Cu) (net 10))
 (segment (start 176.15 76.834) (end 174.625 78.359) (width 1) (layer B.Cu) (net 10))
 (segment (start 194.945 82.677) (end 194.945 88.392) (width 1) (layer B.Cu) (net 10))
 (segment (start 194.182 89.155) (end 192.151 89.155) (width 1) (layer B.Cu) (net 10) (status 20))
 (segment (start 194.945 88.392) (end 194.182 89.155) (width 1) (layer B.Cu) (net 10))
 (segment (start 201.295 86.868) (end 203.962 84.201) (width 1) (layer B.Cu) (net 10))
 (segment (start 224.155 84.201) (end 224.155 81.151) (width 1) (layer B.Cu) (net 10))
 (segment (start 224.155 81.151) (end 221.5515 78.5475) (width 1) (layer B.Cu) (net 10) (status 20))
 (segment (start 201.295 86.868) (end 201.295 90.805) (width 1) (layer B.Cu) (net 10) (status 20))
 (segment (start 202.946 57.404) (end 202.311 57.404) (width 1) (layer B.Cu) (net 10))
 (segment (start 200.279 59.436) (end 200.279 64.01) (width 1) (layer B.Cu) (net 10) (status 20))
 (segment (start 202.311 57.404) (end 200.279 59.436) (width 1) (layer B.Cu) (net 10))
 (segment (start 225.679 54.864) (end 223.139 57.404) (width 1) (layer B.Cu) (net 10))
 (segment (start 225.679 51.7505) (end 225.679 54.864) (width 1) (layer B.Cu) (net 10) (status 10))
 (segment (start 200.279 64.01) (end 200.279 67.183) (width 1) (layer B.Cu) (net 10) (status 10))
 (segment (start 200.279 67.183) (end 197.231 70.231) (width 1) (layer B.Cu) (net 10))
 (segment (start 176.15 76.834) (end 176.15 72.897) (width 1) (layer B.Cu) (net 10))
 (segment (start 178.816 70.231) (end 179.832 70.231) (width 1) (layer B.Cu) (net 10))
 (segment (start 176.15 72.897) (end 178.816 70.231) (width 1) (layer B.Cu) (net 10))
 (segment (start 197.231 70.231) (end 179.832 70.231) (width 1) (layer B.Cu) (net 10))
 (segment (start 223.139 57.404) (end 224.028 57.404) (width 1) (layer B.Cu) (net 10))
 (segment (start 224.028 57.404) (end 225.679 59.055) (width 1) (layer B.Cu) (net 10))
 (segment (start 225.679 74.42) (end 221.5515 78.5475) (width 1) (layer B.Cu) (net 10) (status 20))
 (segment (start 225.679 59.055) (end 225.679 74.42) (width 1) (layer B.Cu) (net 10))
 (segment (start 201.295 90.805) (end 201.295 95.758) (width 1) (layer B.Cu) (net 10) (status 10))
 (segment (start 201.295 95.758) (end 201.93 96.393) (width 1) (layer B.Cu) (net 10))
 (segment (start 224.155 84.201) (end 224.155 94.234) (width 1) (layer B.Cu) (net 10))
 (segment (start 221.996 96.393) (end 201.93 96.393) (width 1) (layer B.Cu) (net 10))
 (segment (start 224.155 94.234) (end 221.996 96.393) (width 1) (layer B.Cu) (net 10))
 (segment (start 181.558 83.906) (end 178.095 83.906) (width 0.25) (layer B.Cu) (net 2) (status 10))
 (segment (start 178.745 83.256) (end 178.095 83.906) (width 0.25) (layer B.Cu) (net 2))
 (segment (start 181.558 83.256) (end 178.745 83.256) (width 0.25) (layer B.Cu) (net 2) (status 10))
 (segment (start 176.911 85.09) (end 178.095 83.906) (width 0.25) (layer B.Cu) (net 2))
 (segment (start 176.911 89.155) (end 176.911 85.09) (width 0.25) (layer B.Cu) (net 2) (status 10))
 (segment (start 210.895 85.557) (end 208.956 85.557) (width 0.25) (layer B.Cu) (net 2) (status 10))
 (segment (start 208.956 85.557) (end 206.375 88.138) (width 0.25) (layer B.Cu) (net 2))
 (segment (start 209.545 84.257) (end 210.895 84.257) (width 0.25) (layer B.Cu) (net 2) (status 20))
 (segment (start 208.33799 83.04999) (end 209.545 84.257) (width 0.25) (layer B.Cu) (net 2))
 (segment (start 208.33799 80.07901) (end 208.33799 83.04999) (width 0.25) (layer B.Cu) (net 2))
 (segment (start 209.8695 78.5475) (end 208.33799 80.07901) (width 0.25) (layer B.Cu) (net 2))
 (segment (start 211.3915 78.5475) (end 209.8695 78.5475) (width 0.25) (layer B.Cu) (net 2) (status 10))
 (segment (start 209.879 56.81) (end 208.448 56.81) (width 0.25) (layer B.Cu) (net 2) (status 10))
 (segment (start 208.448 56.81) (end 207.518 55.88) (width 0.25) (layer B.Cu) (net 2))
 (segment (start 207.518 55.88) (end 207.518 54.483) (width 0.25) (layer B.Cu) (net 2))
 (segment (start 207.518 54.483) (end 208.407 53.594) (width 0.25) (layer B.Cu) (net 2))
 (segment (start 213.6755 53.594) (end 215.519 51.7505) (width 0.25) (layer B.Cu) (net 2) (status 20))
 (segment (start 208.407 53.594) (end 213.6755 53.594) (width 0.25) (layer B.Cu) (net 2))
 (segment (start 209.879 58.76) (end 207.178 58.76) (width 0.25) (layer B.Cu) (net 2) (status 10))
 (segment (start 205.359 60.579) (end 205.359 64.01) (width 0.25) (layer B.Cu) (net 2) (status 20))
 (segment (start 207.178 58.76) (end 205.359 60.579) (width 0.25) (layer B.Cu) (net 2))
 (segment (start 206.375 88.138) (end 206.375 90.805) (width 0.25) (layer B.Cu) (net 2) (status 20))
 (segment (start 197.358 76.834) (end 197.358 74.549) (width 0.25) (layer B.Cu) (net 2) (status 10))
 (segment (start 197.358 74.549) (end 200.914 70.993) (width 0.25) (layer B.Cu) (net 2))
 (segment (start 200.914 70.993) (end 203.581 70.993) (width 0.25) (layer B.Cu) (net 2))
 (segment (start 205.359 69.215) (end 205.359 64.01) (width 0.25) (layer B.Cu) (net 2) (status 20))
 (segment (start 203.581 70.993) (end 205.359 69.215) (width 0.25) (layer B.Cu) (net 2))
 (segment (start 198.374 83.058) (end 198.374 80.391) (width 0.25) (layer B.Cu) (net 2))
 (segment (start 197.358 79.375) (end 197.358 76.834) (width 0.25) (layer B.Cu) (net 2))
 (segment (start 198.374 80.391) (end 197.358 79.375) (width 0.25) (layer B.Cu) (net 2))
 (segment (start 198.247 77.723) (end 197.358 76.834) (width 0.25) (layer B.Cu) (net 2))
 (segment (start 200.406 79.882) (end 198.247 77.723) (width 0.25) (layer B.Cu) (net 2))
 (segment (start 200.406 83.058) (end 200.406 79.882) (width 0.25) (layer B.Cu) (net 2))
 (segment (start 206.375 84.328) (end 206.375 88.138) (width 0.25) (layer B.Cu) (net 2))
 (segment (start 205.105 83.058) (end 206.375 84.328) (width 0.25) (layer B.Cu) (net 2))
 (segment (start 200.406 83.058) (end 205.105 83.058) (width 0.25) (layer B.Cu) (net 2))
 (segment (start 187.758 82.606) (end 189.04841 82.606) (width 0.25) (layer B.Cu) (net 23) (status 10))
 (segment (start 189.04841 82.606) (end 192.278 79.37641) (width 0.25) (layer B.Cu) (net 23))
 (segment (start 192.278 79.37641) (end 192.278 76.834) (width 0.25) (layer B.Cu) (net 23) (status 20))
 (segment (start 217.095 84.257) (end 218.511 84.257) (width 0.25) (layer B.Cu) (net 25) (status 10))
 (segment (start 218.511 84.257) (end 220.091 82.677) (width 0.25) (layer B.Cu) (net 25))
 (segment (start 220.091 82.677) (end 220.091 80.264) (width 0.25) (layer B.Cu) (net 25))
 (segment (start 218.3745 78.5475) (end 216.4715 78.5475) (width 0.25) (layer B.Cu) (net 25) (status 20))
 (segment (start 220.091 80.264) (end 218.3745 78.5475) (width 0.25) (layer B.Cu) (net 25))
 (segment (start 216.079 57.46) (end 219.019 57.46) (width 0.25) (layer B.Cu) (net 26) (status 10))
 (segment (start 220.599 55.88) (end 220.599 51.7505) (width 0.25) (layer B.Cu) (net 26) (status 20))
 (segment (start 219.019 57.46) (end 220.599 55.88) (width 0.25) (layer B.Cu) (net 26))
 (via (at 194.818 73.533) (size 0.8) (drill 0.4) (layers F.Cu B.Cu) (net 5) (status 30))
 (via (at 189.738 73.533) (size 0.8) (drill 0.4) (layers F.Cu B.Cu) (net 5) (status 30))
 (via (at 184.658 73.533) (size 0.8) (drill 0.4) (layers F.Cu B.Cu) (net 8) (status 30))
 (via (at 179.578 73.533) (size 0.8) (drill 0.4) (layers F.Cu B.Cu) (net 4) (status 30))
 (via (at 194.691 92.583) (size 0.8) (drill 0.4) (layers F.Cu B.Cu) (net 6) (status 30))
 (via (at 189.611 92.456) (size 0.8) (drill 0.4) (layers F.Cu B.Cu) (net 6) (status 30))
 (via (at 184.531 92.456) (size 0.8) (drill 0.4) (layers F.Cu B.Cu) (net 9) (status 30))
 (via (at 179.451 92.456) (size 0.8) (drill 0.4) (layers F.Cu B.Cu) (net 7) (status 30))
 (via (at 219.075 94.107) (size 0.8) (drill 0.4) (layers F.Cu B.Cu) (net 13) (status 30))
 (via (at 213.995 94.107) (size 0.8) (drill 0.4) (layers F.Cu B.Cu) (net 16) (status 30))
 (via (at 203.835 94.107) (size 0.8) (drill 0.4) (layers F.Cu B.Cu) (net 14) (status 30))
 (via (at 208.915 94.107) (size 0.8) (drill 0.4) (layers F.Cu B.Cu) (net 14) (status 30))
 (via (at 203.835 75.184) (size 0.8) (drill 0.4) (layers F.Cu B.Cu) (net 11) (status 30))
 (via (at 208.915 75.184) (size 0.8) (drill 0.4) (layers F.Cu B.Cu) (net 11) (status 30))
 (via (at 213.995 75.184) (size 0.8) (drill 0.4) (layers F.Cu B.Cu) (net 15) (status 30))
 (via (at 218.948 75.184) (size 0.8) (drill 0.4) (layers F.Cu B.Cu) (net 12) (status 30))
 (via (at 212.979 67.31) (size 0.8) (drill 0.4) (layers F.Cu B.Cu) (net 17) (status 30))
 (via (at 212.979 48.514) (size 0.8) (drill 0.4) (layers F.Cu B.Cu) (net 18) (status 30))
 (via (at 207.899 67.31) (size 0.8) (drill 0.4) (layers F.Cu B.Cu) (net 19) (status 30))
 (via (at 202.819 67.31) (size 0.8) (drill 0.4) (layers F.Cu B.Cu) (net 19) (status 30))
 (via (at 218.059 67.31) (size 0.8) (drill 0.4) (layers F.Cu B.Cu) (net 20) (status 30))
 (via (at 223.139 48.514) (size 0.8) (drill 0.4) (layers F.Cu B.Cu) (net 21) (status 30))
 (via (at 218.059 48.514) (size 0.8) (drill 0.4) (layers F.Cu B.Cu) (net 21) (status 30))
 (via (at 207.899 48.514) (size 0.8) (drill 0.4) (layers F.Cu B.Cu) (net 22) (status 30))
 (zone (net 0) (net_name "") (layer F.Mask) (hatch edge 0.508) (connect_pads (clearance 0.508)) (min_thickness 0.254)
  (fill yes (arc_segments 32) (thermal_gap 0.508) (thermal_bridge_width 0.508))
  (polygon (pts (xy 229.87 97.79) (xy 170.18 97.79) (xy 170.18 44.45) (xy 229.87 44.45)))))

